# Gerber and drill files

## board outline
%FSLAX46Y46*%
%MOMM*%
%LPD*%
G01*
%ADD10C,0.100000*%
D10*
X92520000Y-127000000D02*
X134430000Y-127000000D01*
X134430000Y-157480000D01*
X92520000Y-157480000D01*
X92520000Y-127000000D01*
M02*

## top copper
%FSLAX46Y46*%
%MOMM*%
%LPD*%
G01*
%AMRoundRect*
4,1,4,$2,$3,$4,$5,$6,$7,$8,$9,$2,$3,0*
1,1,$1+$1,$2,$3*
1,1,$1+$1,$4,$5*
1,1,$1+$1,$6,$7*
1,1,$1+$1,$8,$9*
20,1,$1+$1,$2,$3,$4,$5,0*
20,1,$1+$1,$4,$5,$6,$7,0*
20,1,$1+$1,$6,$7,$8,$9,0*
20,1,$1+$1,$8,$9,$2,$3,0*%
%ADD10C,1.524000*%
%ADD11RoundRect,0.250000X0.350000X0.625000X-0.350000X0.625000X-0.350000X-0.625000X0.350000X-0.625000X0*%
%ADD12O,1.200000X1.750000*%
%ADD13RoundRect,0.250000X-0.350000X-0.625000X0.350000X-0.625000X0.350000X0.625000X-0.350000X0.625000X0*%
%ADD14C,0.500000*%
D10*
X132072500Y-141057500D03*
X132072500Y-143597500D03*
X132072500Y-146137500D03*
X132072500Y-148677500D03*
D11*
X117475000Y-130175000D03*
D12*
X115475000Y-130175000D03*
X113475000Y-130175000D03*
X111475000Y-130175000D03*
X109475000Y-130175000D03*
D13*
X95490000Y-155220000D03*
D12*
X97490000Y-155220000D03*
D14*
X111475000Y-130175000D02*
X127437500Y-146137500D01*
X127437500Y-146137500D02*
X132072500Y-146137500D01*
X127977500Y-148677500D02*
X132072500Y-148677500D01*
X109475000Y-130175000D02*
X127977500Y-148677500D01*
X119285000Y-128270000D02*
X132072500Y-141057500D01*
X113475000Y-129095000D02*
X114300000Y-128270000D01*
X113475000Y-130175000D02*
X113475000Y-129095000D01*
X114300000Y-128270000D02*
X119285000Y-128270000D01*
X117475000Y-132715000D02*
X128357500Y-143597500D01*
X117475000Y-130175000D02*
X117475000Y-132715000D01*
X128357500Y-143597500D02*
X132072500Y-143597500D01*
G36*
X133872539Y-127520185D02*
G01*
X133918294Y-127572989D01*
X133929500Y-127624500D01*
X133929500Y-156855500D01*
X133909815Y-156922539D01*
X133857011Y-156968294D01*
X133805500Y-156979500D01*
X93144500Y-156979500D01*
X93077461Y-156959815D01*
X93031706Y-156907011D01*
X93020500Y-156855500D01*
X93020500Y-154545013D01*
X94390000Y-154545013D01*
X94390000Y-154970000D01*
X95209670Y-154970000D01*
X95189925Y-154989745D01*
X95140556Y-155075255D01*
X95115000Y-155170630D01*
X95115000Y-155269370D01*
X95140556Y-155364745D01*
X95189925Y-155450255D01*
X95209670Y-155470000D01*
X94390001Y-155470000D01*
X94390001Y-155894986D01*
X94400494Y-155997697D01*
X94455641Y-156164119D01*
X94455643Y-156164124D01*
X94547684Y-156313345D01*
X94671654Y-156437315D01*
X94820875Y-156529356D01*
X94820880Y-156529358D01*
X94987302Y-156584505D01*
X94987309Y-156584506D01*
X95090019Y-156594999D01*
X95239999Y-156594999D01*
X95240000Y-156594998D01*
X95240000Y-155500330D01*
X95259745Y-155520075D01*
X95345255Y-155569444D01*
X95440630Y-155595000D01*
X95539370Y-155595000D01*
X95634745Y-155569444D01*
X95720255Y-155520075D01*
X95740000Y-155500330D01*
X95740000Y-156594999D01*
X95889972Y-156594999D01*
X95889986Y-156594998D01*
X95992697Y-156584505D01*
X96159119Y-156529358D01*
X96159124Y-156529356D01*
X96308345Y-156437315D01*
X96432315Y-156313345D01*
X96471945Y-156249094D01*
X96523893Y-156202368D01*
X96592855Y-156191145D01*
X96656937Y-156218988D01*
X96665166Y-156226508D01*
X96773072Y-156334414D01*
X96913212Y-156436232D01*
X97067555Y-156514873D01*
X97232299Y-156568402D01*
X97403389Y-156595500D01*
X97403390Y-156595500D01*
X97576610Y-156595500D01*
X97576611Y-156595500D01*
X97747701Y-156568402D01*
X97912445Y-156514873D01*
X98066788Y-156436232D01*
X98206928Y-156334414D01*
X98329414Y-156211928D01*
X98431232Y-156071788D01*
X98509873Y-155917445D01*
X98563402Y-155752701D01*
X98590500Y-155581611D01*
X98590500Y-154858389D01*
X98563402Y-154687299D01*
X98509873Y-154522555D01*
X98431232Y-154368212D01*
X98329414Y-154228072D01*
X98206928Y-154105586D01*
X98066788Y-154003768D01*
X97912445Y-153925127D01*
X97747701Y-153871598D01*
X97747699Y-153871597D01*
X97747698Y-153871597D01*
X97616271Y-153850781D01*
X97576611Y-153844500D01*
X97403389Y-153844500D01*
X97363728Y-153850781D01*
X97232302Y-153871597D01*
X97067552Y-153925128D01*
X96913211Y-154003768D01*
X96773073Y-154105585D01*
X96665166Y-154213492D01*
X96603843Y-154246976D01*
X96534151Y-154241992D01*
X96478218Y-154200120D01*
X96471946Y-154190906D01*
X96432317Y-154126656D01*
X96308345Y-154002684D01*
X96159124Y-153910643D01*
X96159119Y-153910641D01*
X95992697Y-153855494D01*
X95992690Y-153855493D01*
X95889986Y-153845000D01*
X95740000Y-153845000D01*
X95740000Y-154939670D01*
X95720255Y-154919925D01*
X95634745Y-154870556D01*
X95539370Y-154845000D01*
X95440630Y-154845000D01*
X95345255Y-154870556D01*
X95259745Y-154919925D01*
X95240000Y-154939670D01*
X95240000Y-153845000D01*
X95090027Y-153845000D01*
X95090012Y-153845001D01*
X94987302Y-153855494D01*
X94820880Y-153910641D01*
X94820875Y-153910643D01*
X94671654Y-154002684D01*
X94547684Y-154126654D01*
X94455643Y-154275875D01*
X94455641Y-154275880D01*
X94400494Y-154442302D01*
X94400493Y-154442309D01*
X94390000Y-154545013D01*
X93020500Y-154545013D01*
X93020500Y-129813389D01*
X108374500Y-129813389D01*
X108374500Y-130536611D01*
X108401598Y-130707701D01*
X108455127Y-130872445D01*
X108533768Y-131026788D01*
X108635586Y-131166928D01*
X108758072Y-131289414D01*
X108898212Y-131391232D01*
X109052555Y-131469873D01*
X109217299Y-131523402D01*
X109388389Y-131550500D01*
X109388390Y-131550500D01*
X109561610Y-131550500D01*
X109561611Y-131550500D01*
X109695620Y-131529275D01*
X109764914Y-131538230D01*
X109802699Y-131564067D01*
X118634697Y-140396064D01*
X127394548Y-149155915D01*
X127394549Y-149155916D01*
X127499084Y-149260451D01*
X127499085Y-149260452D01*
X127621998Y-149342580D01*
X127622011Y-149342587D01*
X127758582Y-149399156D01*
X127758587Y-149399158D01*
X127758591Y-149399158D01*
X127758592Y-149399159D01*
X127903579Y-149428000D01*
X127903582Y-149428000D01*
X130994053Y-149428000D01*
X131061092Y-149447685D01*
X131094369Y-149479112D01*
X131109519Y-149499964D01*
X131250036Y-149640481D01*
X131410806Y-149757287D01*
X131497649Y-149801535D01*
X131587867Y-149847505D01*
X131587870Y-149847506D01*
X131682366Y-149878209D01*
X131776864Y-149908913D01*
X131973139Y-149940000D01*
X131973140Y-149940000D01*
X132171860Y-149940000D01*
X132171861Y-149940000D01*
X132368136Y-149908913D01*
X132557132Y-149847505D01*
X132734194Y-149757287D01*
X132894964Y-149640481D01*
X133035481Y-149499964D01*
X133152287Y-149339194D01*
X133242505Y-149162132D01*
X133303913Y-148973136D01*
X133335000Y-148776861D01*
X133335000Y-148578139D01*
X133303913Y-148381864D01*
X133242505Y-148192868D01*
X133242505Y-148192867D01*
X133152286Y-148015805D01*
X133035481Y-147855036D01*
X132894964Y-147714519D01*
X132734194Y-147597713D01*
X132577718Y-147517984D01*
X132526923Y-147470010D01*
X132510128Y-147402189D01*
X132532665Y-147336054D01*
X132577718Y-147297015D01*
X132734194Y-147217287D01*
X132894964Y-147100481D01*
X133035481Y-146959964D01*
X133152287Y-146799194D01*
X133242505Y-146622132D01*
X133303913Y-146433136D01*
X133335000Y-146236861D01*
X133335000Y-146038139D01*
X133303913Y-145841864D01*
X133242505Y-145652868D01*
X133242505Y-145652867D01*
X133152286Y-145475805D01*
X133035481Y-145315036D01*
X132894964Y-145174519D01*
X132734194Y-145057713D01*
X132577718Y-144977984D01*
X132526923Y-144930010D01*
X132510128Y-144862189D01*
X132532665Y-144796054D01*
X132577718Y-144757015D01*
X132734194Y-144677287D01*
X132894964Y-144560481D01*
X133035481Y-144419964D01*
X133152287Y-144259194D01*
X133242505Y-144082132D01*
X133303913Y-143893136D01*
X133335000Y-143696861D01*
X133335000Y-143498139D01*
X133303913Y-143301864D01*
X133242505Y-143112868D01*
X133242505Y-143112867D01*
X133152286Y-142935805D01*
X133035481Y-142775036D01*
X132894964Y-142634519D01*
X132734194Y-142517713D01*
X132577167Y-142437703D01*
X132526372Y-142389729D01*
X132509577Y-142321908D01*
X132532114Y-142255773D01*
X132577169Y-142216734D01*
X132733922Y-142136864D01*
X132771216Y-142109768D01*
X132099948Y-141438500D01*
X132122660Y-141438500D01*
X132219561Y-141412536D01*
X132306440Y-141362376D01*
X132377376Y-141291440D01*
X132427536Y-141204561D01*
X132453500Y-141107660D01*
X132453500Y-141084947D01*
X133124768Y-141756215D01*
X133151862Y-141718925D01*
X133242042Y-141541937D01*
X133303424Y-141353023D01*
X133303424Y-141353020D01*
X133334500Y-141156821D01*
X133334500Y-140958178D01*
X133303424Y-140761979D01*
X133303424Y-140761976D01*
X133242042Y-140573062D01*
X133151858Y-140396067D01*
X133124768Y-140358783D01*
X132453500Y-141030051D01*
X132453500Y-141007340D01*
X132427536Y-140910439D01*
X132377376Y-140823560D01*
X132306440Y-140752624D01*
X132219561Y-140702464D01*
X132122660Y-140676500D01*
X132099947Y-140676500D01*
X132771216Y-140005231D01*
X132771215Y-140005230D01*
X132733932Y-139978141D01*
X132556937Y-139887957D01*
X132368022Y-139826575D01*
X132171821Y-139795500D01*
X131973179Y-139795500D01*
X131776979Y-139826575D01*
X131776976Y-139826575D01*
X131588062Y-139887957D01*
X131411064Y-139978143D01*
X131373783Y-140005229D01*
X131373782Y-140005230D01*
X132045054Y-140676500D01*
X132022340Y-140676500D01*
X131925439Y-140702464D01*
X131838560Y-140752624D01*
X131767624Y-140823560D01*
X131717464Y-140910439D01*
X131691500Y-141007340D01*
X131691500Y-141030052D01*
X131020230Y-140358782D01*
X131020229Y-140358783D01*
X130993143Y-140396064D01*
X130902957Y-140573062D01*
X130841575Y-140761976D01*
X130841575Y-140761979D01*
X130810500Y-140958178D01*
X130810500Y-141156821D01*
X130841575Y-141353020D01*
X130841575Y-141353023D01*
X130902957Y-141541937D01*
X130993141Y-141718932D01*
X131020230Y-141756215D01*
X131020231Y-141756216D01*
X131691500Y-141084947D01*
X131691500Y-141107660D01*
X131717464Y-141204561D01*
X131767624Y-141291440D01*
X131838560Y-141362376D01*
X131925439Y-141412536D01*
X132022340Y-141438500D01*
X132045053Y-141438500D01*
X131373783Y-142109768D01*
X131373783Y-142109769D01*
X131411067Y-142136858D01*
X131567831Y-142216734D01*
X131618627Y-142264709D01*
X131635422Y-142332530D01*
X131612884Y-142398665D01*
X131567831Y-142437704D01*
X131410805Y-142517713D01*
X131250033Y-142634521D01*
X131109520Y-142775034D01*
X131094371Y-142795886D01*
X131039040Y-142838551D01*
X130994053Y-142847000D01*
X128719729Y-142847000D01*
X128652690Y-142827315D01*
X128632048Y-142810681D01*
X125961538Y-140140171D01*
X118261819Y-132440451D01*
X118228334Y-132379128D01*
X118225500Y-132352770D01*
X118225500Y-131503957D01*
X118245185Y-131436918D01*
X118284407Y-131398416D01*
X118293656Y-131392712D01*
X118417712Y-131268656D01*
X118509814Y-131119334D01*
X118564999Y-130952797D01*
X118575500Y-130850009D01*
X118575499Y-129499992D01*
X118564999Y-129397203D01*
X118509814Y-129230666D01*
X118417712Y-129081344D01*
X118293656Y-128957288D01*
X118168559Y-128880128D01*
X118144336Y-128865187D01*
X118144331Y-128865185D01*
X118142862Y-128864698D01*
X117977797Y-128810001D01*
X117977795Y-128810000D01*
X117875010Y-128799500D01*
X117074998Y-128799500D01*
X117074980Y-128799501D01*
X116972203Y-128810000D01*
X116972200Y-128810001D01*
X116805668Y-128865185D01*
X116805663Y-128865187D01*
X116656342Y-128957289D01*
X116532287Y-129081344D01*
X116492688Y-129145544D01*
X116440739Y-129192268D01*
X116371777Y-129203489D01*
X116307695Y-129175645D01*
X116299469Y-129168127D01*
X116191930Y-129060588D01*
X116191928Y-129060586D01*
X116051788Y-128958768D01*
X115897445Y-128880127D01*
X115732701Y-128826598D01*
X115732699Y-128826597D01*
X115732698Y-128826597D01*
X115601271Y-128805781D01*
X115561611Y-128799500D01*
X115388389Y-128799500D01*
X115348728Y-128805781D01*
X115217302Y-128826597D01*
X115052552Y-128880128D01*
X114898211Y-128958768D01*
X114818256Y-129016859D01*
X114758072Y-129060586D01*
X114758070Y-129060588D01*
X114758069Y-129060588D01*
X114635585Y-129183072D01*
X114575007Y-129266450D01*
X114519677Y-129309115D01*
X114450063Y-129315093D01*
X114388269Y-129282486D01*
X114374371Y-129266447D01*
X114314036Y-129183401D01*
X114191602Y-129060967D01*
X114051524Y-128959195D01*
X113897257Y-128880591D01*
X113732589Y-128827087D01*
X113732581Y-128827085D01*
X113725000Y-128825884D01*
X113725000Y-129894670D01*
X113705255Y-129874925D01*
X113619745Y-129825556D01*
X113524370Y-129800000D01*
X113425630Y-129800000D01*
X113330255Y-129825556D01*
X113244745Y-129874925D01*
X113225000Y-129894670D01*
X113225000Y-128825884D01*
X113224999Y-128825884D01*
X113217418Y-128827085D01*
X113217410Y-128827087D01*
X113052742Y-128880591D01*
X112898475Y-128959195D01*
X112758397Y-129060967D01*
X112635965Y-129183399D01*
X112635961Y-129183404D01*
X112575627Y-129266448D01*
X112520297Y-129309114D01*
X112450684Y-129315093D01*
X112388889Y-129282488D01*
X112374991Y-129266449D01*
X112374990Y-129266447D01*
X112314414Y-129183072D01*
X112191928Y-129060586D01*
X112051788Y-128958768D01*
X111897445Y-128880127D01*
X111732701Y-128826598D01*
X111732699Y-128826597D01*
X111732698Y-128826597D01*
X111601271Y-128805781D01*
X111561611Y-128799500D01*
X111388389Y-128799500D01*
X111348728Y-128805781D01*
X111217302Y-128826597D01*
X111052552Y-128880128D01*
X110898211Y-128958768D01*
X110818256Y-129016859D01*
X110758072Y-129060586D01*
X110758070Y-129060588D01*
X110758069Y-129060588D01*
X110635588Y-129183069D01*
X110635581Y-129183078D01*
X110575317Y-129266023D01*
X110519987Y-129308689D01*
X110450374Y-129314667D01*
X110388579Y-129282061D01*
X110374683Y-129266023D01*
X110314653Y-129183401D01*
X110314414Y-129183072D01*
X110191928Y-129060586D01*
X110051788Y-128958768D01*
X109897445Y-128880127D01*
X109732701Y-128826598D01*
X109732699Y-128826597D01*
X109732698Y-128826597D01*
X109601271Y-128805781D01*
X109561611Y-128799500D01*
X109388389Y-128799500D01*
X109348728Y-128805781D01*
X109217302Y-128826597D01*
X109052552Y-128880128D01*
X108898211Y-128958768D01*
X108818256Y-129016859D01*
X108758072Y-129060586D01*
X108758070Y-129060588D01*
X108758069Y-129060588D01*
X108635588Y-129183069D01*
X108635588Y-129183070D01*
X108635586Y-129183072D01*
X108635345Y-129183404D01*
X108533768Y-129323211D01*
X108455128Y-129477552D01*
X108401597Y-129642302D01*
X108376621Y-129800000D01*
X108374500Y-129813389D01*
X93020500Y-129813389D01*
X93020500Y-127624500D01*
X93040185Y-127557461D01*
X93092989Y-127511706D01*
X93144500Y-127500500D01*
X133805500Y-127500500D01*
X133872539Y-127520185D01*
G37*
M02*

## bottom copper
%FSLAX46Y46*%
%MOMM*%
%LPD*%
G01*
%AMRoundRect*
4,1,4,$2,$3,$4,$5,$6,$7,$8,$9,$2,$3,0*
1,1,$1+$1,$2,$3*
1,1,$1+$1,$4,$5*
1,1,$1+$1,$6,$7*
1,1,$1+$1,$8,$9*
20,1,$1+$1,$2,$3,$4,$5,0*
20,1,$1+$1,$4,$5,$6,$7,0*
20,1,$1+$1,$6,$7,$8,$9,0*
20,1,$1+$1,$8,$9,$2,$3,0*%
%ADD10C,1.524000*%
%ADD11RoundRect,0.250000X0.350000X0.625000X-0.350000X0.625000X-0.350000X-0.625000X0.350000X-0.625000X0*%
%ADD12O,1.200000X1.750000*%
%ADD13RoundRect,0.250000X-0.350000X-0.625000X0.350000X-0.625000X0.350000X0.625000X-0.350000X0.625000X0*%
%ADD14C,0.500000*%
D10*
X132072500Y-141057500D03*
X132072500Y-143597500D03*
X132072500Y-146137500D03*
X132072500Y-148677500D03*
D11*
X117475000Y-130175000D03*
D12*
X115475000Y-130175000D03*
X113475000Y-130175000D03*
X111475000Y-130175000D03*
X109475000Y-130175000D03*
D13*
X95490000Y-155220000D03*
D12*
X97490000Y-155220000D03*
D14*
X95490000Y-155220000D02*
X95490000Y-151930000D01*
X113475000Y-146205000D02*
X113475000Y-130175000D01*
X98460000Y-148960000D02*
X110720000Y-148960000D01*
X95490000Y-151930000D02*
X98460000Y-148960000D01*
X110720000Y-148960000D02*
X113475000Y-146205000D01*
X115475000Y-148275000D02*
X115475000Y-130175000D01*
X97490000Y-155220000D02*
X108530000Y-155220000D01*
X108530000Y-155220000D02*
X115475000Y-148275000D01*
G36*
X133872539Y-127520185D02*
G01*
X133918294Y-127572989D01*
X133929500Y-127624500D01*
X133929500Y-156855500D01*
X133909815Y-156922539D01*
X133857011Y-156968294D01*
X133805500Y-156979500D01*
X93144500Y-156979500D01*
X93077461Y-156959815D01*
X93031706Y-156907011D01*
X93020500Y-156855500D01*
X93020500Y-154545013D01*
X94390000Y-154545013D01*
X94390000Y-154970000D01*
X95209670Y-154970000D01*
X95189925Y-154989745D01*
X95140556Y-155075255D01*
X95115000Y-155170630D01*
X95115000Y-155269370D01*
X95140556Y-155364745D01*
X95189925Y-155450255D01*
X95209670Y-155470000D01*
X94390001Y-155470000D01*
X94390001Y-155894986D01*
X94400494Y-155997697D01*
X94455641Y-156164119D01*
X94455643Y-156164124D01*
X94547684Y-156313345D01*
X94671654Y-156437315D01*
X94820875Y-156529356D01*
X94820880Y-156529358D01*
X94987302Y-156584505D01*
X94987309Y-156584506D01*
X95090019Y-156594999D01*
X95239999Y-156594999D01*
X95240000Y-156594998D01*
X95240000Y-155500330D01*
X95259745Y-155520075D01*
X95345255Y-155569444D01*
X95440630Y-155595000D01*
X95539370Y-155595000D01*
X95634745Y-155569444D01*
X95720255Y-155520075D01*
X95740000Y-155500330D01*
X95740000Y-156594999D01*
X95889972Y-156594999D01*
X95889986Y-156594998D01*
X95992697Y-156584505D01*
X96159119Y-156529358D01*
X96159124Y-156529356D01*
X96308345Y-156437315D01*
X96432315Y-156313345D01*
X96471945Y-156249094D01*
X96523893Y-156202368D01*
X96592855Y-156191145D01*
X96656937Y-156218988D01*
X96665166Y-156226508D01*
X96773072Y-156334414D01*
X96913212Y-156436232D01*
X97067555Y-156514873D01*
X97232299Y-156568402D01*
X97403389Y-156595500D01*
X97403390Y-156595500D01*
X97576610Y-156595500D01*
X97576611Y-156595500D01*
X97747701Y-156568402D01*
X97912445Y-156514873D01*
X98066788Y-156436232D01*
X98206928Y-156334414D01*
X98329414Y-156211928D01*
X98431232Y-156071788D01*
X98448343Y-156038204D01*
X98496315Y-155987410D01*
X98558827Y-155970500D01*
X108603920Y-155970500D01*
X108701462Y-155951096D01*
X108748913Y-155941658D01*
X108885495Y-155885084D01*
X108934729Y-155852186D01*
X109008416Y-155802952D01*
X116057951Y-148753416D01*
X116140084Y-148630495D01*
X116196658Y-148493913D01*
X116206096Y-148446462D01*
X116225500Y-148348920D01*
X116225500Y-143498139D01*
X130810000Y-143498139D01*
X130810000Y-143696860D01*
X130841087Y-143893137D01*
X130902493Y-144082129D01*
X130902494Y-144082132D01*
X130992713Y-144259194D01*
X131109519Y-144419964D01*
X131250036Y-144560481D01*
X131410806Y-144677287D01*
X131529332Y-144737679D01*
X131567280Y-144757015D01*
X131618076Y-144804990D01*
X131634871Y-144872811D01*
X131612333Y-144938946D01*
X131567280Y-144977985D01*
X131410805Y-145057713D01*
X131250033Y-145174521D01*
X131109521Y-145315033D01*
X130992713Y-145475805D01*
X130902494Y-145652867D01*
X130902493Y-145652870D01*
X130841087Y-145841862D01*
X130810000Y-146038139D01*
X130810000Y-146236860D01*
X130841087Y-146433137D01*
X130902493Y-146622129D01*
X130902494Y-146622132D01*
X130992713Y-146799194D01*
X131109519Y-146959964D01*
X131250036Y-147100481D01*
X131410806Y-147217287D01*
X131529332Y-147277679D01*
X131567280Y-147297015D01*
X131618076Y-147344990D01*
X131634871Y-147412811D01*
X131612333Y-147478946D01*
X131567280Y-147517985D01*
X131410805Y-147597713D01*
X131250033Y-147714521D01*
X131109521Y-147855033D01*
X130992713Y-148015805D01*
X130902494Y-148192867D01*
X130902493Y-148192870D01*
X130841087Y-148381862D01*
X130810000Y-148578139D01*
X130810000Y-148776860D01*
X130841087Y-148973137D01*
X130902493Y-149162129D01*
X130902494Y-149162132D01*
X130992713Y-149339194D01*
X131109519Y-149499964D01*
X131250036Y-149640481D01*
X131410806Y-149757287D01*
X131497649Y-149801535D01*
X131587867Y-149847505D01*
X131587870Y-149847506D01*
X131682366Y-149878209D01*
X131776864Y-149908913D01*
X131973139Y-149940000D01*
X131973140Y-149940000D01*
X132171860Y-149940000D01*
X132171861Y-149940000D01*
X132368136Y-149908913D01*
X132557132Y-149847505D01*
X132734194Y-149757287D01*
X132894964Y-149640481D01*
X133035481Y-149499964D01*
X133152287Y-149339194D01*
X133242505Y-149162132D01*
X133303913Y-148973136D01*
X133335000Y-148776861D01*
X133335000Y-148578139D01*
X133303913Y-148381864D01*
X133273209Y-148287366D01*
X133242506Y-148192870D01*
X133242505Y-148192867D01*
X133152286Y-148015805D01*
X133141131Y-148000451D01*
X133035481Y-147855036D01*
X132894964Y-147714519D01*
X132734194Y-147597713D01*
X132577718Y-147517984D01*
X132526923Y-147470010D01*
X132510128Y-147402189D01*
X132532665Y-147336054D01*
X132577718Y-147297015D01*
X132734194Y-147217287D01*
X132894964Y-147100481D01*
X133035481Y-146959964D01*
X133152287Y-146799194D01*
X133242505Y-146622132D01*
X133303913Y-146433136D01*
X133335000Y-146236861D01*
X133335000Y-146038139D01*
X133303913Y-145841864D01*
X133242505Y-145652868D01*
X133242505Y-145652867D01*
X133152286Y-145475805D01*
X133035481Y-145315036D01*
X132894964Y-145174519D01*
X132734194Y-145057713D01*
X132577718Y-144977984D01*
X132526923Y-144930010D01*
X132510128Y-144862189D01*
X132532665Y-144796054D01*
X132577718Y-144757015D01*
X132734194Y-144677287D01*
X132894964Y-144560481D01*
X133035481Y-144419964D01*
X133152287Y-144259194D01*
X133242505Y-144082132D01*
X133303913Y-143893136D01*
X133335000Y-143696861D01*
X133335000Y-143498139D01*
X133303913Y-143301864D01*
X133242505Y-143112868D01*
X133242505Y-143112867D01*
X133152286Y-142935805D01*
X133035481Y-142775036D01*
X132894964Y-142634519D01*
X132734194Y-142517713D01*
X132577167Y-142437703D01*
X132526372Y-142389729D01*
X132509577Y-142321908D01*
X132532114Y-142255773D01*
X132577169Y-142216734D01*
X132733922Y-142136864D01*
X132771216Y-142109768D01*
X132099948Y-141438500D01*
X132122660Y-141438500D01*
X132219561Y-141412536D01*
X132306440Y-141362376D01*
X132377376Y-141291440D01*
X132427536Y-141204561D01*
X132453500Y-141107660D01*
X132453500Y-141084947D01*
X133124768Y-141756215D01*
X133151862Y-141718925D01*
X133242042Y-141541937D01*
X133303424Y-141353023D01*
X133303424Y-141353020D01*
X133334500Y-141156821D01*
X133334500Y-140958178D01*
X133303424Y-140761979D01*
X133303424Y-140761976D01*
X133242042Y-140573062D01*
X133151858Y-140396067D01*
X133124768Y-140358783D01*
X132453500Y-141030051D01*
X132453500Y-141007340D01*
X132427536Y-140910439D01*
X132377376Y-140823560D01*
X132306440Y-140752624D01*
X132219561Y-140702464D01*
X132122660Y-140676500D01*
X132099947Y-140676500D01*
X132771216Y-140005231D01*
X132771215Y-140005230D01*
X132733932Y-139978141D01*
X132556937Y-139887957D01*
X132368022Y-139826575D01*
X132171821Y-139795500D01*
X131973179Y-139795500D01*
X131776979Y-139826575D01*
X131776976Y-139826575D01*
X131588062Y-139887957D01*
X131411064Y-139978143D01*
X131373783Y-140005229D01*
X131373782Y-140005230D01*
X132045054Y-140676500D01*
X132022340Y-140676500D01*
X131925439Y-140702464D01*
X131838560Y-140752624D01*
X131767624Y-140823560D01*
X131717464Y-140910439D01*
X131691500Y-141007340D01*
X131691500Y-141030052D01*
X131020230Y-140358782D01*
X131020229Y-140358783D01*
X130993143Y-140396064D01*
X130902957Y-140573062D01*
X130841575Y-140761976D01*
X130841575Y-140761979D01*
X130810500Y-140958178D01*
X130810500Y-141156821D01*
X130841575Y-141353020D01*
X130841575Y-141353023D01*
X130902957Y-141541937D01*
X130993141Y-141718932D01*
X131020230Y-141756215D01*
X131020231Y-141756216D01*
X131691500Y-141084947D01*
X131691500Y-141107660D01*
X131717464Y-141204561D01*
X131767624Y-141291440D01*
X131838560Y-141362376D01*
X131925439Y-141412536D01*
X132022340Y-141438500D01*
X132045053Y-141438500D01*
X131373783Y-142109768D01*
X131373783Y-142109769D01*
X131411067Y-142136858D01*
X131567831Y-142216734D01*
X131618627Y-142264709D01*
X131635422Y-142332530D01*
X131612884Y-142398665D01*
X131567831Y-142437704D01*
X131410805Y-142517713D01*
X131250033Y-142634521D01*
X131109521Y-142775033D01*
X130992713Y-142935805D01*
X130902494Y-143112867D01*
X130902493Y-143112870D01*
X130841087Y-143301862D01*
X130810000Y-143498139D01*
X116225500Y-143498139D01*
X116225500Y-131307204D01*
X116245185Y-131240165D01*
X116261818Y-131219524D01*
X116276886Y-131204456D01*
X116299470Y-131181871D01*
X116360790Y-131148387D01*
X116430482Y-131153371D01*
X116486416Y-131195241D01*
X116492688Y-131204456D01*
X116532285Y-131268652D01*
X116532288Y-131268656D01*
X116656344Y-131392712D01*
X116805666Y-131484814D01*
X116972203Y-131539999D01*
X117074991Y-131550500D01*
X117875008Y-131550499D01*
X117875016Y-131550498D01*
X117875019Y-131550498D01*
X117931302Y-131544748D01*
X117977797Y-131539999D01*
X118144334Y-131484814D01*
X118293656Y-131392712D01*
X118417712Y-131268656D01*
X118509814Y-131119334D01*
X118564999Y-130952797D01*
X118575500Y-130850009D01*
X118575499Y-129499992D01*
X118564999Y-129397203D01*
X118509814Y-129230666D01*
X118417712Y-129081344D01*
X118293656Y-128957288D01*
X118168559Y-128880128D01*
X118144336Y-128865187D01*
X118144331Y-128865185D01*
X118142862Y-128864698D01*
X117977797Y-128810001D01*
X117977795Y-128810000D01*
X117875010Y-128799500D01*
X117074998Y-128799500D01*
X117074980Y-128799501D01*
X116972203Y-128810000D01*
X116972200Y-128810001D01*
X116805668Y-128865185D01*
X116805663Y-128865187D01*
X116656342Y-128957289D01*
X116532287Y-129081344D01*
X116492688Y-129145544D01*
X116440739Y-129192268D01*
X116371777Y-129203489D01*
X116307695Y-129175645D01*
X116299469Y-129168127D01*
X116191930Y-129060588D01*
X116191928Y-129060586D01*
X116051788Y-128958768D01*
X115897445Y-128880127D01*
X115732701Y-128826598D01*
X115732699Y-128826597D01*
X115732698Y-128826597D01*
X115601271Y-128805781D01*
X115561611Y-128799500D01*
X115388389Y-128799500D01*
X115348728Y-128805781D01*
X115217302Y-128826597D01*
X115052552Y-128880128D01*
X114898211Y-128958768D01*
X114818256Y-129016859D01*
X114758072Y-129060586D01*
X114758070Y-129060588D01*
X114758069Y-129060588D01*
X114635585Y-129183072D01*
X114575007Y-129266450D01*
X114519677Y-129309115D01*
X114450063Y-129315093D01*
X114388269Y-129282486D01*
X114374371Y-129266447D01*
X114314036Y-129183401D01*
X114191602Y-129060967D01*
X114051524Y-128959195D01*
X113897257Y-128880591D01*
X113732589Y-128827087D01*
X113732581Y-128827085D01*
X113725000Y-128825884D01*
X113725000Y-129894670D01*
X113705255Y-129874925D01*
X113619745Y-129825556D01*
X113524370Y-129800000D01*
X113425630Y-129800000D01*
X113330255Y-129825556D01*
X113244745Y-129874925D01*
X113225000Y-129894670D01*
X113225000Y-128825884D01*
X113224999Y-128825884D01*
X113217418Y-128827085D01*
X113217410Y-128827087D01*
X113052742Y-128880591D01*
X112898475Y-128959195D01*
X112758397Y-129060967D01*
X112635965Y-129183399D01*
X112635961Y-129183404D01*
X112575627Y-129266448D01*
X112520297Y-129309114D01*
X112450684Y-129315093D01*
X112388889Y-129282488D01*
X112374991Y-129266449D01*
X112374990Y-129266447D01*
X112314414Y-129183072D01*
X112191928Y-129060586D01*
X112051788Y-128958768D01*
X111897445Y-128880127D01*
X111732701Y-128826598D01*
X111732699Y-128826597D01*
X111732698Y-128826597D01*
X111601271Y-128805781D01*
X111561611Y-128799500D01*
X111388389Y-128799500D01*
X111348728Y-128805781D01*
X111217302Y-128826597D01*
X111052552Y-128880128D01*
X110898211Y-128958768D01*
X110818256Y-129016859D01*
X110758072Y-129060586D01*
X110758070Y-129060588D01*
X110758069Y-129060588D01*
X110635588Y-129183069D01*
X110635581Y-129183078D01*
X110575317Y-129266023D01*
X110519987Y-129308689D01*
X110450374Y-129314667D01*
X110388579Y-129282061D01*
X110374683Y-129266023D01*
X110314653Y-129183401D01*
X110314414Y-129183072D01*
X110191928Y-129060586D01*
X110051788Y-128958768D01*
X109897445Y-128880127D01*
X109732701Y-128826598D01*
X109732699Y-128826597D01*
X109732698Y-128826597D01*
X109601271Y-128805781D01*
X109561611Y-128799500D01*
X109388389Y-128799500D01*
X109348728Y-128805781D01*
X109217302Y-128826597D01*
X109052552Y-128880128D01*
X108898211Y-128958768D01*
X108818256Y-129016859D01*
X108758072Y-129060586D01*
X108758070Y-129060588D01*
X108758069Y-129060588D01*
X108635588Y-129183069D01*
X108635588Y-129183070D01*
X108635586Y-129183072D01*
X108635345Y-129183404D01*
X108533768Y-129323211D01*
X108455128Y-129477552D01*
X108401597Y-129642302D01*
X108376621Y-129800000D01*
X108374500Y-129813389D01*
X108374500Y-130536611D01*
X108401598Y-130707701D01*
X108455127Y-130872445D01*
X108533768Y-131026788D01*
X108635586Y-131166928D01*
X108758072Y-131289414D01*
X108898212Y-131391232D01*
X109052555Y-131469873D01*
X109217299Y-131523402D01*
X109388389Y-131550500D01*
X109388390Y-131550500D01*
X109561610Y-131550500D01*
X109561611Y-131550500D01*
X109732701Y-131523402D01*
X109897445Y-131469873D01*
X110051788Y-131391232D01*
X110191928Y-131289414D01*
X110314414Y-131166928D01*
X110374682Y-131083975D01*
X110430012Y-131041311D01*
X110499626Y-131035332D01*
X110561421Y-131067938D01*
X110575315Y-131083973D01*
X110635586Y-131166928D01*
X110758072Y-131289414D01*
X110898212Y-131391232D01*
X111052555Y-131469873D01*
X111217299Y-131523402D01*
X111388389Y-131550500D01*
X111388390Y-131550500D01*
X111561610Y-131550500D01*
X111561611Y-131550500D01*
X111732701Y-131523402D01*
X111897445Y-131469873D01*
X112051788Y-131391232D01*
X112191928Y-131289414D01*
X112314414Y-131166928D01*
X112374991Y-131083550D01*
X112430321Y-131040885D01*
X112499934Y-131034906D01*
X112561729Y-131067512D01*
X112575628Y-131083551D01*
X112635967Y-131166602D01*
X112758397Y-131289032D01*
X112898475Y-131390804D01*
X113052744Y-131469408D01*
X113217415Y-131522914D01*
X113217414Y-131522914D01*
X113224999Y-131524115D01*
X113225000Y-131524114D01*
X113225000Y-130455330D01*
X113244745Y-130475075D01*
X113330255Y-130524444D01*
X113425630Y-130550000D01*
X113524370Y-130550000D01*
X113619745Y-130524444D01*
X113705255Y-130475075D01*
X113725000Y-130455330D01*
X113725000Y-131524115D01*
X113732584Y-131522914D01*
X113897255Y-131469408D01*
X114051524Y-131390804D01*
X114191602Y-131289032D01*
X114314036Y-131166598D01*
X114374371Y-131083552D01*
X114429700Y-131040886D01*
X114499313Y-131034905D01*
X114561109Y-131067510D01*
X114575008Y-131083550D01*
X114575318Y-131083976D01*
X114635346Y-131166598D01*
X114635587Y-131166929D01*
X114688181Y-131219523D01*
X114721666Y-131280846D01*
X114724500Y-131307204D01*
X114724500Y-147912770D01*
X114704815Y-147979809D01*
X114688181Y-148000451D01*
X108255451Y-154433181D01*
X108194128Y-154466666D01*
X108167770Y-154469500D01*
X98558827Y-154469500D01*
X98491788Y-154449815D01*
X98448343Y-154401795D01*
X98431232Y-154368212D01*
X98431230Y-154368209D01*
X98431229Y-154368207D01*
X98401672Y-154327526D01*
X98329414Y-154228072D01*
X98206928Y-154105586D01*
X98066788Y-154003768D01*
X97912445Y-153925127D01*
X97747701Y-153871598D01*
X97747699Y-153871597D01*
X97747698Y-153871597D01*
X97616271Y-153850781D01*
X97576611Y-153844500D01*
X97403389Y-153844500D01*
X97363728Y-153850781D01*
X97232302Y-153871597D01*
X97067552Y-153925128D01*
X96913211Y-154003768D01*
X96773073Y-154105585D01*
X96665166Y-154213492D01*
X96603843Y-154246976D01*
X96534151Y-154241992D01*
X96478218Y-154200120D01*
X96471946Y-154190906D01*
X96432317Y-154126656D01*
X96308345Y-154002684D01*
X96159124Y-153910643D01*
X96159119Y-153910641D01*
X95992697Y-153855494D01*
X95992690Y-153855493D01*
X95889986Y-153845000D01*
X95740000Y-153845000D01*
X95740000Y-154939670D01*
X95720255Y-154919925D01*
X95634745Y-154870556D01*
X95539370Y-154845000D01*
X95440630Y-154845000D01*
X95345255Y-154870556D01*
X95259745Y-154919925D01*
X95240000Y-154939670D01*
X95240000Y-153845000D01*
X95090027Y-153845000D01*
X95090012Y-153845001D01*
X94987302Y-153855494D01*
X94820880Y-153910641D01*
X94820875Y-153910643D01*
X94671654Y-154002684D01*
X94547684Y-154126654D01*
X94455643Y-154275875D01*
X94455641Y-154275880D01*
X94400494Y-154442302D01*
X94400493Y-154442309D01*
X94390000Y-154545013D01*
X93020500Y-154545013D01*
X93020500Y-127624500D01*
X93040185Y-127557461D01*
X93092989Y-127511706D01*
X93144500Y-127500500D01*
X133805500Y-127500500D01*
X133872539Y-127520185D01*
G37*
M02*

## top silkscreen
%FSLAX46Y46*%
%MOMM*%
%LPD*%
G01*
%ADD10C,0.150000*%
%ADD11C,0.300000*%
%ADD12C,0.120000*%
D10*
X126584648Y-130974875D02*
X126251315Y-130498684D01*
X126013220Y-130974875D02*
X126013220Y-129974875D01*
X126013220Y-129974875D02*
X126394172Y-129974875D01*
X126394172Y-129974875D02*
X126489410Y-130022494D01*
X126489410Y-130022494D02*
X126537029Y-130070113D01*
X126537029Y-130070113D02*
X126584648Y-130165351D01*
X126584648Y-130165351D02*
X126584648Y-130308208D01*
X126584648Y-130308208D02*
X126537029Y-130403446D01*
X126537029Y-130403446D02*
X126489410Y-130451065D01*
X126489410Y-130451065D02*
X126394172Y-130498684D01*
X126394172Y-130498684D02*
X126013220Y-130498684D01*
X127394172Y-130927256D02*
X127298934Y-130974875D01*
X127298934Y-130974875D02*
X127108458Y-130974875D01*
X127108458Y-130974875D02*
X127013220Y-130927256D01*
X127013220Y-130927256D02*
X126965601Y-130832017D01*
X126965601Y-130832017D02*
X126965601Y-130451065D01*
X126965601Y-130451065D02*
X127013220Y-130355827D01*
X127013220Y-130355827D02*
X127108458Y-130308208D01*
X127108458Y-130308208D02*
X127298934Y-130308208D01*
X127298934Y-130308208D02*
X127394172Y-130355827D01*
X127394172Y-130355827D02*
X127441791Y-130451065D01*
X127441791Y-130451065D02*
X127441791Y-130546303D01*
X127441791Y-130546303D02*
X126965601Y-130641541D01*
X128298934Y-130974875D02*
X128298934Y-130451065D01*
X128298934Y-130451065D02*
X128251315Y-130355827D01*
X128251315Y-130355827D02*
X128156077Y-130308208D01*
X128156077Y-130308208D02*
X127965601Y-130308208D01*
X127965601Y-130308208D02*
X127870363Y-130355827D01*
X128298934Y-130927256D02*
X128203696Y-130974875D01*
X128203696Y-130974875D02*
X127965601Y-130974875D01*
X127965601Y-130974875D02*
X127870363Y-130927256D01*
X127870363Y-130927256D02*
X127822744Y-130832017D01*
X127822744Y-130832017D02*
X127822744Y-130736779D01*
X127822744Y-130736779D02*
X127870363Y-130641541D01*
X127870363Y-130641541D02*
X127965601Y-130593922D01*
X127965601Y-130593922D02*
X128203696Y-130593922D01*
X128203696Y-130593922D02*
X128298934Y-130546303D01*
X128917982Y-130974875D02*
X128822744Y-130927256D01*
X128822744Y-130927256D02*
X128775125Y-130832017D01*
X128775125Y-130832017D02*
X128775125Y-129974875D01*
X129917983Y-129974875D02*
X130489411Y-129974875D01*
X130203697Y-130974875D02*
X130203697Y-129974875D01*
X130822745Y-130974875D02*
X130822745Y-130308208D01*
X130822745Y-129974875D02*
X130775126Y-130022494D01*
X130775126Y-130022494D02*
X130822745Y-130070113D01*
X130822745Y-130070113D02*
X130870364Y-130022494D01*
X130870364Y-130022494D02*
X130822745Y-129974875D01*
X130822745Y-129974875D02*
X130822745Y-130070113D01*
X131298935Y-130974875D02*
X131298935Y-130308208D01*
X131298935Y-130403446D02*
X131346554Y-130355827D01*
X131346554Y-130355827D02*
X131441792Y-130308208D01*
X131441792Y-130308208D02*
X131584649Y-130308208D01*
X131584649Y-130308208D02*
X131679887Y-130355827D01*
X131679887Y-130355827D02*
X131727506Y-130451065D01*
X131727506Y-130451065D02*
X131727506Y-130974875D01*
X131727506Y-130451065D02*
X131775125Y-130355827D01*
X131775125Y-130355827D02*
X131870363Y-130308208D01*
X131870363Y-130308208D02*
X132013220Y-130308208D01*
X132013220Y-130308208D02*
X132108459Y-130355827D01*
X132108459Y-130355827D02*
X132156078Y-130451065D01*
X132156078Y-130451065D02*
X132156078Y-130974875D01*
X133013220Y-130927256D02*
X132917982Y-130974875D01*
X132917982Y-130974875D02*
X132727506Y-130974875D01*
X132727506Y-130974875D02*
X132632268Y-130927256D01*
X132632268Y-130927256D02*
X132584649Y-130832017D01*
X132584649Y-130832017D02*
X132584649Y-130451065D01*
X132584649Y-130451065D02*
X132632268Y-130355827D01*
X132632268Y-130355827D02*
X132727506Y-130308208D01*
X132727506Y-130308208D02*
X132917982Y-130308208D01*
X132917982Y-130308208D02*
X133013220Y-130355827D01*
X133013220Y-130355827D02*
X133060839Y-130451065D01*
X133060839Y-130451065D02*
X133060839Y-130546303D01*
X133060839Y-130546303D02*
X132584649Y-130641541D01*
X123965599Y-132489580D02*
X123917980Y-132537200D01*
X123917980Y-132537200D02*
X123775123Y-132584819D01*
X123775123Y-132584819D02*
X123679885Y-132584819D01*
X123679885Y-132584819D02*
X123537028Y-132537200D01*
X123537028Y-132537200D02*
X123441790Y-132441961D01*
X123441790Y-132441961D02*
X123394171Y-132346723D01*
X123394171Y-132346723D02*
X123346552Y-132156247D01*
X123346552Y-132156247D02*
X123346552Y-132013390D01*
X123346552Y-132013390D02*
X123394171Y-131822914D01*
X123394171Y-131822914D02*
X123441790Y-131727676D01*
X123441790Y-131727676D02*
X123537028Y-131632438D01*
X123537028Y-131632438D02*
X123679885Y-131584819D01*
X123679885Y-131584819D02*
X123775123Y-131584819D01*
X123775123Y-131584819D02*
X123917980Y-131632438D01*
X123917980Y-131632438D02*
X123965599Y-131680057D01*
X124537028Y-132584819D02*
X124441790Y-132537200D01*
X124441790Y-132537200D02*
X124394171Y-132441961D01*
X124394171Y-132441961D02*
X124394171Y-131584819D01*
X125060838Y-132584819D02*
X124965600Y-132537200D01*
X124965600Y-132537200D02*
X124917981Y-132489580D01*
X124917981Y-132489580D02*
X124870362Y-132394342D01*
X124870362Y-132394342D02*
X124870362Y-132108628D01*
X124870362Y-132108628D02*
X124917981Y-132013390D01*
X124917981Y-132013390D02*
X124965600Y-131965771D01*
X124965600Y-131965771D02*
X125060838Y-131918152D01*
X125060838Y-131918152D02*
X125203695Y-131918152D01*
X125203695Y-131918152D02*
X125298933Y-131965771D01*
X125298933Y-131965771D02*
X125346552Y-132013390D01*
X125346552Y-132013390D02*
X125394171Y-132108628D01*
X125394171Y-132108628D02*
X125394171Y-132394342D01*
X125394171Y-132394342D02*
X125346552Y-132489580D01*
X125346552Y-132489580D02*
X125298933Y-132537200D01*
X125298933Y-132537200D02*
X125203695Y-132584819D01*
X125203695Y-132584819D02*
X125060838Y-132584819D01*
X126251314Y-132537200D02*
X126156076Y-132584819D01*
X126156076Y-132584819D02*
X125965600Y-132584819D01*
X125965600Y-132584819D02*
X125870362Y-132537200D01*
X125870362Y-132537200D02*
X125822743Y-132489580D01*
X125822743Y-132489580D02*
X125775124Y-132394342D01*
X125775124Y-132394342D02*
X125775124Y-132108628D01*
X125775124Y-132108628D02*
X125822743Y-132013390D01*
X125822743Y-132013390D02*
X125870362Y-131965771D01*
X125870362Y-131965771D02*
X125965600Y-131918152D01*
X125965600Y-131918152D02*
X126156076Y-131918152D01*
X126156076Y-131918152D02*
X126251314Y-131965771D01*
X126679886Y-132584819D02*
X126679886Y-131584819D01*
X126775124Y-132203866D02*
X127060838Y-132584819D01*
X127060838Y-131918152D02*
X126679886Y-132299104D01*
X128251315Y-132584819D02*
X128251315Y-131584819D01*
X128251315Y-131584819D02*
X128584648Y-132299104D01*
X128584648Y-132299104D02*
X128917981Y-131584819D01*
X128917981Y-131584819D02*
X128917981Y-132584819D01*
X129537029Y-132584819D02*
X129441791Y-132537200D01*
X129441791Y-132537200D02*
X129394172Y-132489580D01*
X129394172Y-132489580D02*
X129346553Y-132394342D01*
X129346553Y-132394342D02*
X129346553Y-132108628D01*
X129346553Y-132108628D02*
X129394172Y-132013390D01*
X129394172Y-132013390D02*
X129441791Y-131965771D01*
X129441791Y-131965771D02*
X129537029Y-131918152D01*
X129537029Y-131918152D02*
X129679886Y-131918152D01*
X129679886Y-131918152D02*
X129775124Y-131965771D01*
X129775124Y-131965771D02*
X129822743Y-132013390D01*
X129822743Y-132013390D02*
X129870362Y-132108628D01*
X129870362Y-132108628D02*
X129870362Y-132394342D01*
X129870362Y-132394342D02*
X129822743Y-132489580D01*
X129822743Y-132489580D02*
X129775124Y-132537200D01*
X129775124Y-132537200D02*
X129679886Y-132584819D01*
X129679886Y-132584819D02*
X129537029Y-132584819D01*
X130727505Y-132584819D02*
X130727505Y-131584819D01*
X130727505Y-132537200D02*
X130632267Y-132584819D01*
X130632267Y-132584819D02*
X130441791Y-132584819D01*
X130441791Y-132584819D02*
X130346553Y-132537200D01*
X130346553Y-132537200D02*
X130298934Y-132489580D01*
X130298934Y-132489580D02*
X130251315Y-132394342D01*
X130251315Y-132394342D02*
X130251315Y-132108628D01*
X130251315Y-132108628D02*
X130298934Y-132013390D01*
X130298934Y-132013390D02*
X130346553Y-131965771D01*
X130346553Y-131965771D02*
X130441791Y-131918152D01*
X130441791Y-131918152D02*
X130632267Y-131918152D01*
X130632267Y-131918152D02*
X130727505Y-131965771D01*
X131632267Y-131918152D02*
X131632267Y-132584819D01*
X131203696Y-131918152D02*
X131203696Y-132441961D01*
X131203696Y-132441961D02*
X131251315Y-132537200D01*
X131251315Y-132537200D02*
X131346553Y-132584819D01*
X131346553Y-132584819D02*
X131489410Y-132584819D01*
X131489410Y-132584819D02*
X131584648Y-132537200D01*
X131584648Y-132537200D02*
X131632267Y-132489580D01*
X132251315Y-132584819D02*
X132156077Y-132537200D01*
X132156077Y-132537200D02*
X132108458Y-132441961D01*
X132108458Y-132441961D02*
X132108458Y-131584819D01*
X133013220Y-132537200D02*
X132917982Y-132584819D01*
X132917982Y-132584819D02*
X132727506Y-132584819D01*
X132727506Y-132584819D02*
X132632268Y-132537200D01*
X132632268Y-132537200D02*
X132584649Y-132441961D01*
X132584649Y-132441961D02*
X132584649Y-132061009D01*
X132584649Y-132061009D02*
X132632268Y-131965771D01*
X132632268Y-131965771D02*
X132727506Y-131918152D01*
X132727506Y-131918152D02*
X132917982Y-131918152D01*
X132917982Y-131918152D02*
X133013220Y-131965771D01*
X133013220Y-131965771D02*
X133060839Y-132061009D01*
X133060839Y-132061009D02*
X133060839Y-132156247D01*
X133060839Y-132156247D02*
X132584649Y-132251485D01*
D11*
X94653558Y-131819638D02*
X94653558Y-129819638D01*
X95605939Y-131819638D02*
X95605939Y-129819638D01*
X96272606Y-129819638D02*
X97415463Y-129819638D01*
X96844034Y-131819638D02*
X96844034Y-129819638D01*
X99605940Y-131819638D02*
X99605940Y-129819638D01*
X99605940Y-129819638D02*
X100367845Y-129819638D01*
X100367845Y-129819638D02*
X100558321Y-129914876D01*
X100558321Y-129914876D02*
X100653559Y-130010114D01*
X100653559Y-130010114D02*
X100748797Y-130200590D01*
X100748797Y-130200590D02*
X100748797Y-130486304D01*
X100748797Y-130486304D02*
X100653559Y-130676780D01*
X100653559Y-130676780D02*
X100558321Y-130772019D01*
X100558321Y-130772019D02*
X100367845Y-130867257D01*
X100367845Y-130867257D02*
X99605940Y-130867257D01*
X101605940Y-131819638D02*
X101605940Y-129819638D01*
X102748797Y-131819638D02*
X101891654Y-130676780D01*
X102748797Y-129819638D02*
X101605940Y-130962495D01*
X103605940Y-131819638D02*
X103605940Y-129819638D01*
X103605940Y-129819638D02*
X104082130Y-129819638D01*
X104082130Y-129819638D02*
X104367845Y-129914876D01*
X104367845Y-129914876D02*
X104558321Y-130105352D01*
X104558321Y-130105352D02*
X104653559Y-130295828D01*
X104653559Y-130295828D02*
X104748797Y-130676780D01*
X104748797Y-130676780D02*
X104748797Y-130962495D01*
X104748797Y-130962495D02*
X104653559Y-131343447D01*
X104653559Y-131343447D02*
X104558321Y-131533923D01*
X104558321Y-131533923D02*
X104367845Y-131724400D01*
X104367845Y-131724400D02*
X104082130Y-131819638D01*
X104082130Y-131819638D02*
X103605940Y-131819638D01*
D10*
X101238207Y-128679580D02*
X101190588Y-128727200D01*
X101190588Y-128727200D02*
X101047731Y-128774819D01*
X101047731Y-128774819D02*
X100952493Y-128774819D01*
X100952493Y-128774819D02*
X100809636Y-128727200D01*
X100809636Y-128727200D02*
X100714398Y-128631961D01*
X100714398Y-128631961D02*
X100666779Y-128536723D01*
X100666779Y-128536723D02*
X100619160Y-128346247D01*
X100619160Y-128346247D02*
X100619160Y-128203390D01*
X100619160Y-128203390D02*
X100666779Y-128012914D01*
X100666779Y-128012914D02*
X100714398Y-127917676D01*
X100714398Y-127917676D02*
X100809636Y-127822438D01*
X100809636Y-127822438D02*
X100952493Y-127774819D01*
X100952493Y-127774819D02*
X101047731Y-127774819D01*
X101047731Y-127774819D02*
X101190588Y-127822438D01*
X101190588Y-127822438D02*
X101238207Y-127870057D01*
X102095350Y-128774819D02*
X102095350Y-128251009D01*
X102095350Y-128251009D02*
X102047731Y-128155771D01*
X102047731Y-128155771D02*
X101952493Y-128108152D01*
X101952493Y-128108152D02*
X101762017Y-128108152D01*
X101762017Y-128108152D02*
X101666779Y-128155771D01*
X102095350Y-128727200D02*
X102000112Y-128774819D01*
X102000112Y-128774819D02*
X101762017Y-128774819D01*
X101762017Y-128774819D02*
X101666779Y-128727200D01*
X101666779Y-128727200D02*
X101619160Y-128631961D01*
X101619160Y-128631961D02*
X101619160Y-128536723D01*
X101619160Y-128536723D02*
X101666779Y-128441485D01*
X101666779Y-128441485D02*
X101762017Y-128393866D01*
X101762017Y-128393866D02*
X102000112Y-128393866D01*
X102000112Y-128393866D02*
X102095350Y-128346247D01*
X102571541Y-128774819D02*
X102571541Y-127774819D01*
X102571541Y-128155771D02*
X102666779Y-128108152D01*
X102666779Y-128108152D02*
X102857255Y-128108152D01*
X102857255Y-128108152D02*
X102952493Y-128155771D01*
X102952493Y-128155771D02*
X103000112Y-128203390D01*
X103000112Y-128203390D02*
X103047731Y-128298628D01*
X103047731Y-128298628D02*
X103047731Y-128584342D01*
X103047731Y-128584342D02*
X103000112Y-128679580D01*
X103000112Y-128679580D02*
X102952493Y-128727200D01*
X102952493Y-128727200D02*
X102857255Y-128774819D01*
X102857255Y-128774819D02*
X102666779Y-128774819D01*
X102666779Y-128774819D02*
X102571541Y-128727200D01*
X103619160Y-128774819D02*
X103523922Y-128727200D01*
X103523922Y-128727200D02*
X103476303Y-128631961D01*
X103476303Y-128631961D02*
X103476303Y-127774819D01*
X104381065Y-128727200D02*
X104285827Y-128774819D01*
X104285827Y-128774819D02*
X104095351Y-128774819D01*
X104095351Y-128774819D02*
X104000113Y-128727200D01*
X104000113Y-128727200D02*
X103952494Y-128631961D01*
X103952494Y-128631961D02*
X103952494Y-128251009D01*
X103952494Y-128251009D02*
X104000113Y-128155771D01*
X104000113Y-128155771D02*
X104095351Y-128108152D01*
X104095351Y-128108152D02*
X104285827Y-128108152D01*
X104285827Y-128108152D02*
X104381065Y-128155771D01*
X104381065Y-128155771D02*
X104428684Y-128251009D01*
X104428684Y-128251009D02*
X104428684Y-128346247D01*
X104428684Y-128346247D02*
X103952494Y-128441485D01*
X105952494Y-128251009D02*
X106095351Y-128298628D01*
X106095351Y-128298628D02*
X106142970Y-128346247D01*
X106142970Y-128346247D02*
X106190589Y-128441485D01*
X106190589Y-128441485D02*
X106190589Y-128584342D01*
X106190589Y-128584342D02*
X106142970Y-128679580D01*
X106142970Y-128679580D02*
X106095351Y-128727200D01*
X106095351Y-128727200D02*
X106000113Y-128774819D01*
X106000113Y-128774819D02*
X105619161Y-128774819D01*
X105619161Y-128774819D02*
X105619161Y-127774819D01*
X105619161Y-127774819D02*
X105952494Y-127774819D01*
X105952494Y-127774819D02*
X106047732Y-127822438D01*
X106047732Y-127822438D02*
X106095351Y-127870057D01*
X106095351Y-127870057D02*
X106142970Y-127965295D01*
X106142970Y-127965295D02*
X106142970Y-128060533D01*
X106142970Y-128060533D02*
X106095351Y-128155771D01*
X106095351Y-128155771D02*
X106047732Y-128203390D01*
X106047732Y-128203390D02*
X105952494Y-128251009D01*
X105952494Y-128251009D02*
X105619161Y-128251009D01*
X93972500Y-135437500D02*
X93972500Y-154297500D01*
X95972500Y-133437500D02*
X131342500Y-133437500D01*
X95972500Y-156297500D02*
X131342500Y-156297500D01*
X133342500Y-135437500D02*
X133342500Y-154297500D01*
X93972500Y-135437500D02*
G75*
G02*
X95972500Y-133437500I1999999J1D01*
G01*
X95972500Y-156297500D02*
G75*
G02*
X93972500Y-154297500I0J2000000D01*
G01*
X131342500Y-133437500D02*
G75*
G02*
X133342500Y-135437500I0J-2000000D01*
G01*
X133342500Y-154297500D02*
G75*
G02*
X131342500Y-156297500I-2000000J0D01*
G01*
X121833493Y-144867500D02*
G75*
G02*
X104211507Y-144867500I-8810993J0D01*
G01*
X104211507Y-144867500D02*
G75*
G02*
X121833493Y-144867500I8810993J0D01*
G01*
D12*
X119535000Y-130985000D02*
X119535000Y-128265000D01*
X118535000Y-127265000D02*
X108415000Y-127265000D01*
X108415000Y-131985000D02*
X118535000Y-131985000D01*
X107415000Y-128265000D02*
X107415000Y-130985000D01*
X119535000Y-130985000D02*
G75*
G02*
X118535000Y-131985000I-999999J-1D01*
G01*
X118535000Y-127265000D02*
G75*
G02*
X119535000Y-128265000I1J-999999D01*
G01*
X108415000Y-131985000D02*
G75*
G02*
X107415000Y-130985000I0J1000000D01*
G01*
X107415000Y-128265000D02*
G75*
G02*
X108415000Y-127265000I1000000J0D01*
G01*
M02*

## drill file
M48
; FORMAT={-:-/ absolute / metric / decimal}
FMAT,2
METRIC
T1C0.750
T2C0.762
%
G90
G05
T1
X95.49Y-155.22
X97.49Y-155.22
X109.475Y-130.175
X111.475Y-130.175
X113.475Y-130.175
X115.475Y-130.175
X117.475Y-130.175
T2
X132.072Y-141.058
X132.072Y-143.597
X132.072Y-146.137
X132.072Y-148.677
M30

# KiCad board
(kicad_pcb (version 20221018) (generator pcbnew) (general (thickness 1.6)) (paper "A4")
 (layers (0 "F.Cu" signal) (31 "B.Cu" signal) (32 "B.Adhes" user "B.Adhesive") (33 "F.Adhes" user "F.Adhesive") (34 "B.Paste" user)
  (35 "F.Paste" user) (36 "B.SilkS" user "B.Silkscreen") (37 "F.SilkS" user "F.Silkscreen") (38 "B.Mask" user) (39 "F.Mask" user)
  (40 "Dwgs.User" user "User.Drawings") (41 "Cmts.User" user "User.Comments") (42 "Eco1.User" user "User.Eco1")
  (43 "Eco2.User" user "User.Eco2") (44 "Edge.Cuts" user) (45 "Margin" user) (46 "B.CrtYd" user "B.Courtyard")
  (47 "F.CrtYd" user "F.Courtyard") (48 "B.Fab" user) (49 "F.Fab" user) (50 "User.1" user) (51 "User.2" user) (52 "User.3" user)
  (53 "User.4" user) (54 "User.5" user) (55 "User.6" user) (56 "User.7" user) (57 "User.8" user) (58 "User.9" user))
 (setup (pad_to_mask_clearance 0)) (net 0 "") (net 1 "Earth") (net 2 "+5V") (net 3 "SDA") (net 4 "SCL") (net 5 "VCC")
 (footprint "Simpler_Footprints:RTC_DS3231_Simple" (layer "F.Cu") (at 93.9725 133.4375)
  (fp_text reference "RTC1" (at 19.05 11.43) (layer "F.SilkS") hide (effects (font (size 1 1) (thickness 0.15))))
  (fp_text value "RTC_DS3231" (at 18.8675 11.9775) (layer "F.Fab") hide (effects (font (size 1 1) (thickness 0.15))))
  (fp_line (start 0 2) (end 0 20.86) (stroke (width 0.15) (type solid)) (layer "F.SilkS"))
  (fp_line (start 2 0) (end 37.37 0) (stroke (width 0.15) (type solid)) (layer "F.SilkS"))
  (fp_line (start 2 22.86) (end 37.37 22.86) (stroke (width 0.15) (type solid)) (layer "F.SilkS"))
  (fp_line (start 39.37 2) (end 39.37 20.86) (stroke (width 0.15) (type solid)) (layer "F.SilkS"))
  (fp_arc (start 0 2) (mid 0.585786 0.585786) (end 2 0) (stroke (width 0.15) (type default)) (layer "F.SilkS"))
  (fp_arc (start 2 22.86) (mid 0.585786 22.274214) (end 0 20.86) (stroke (width 0.15) (type default)) (layer "F.SilkS"))
  (fp_arc (start 37.37 0) (mid 38.784214 0.585786) (end 39.37 2) (stroke (width 0.15) (type default)) (layer "F.SilkS"))
  (fp_arc (start 39.37 20.86) (mid 38.784214 22.274214) (end 37.37 22.86) (stroke (width 0.15) (type default)) (layer "F.SilkS"))
  (fp_circle (center 19.05 11.43) (end 27.860993 11.43) (stroke (width 0.15) (type default)) (fill none) (layer "F.SilkS"))
  (pad "1" thru_hole circle (at 38.1 7.62) (size 1.524 1.524) (drill 0.762) (layers "*.Cu" "*.Mask") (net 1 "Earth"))
  (pad "2" thru_hole circle (at 38.1 10.16) (size 1.524 1.524) (drill 0.762) (layers "*.Cu" "*.Mask") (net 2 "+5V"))
  (pad "3" thru_hole circle (at 38.1 12.7) (size 1.524 1.524) (drill 0.762) (layers "*.Cu" "*.Mask") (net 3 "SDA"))
  (pad "4" thru_hole circle (at 38.1 15.24) (size 1.524 1.524) (drill 0.762) (layers "*.Cu" "*.Mask") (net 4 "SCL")))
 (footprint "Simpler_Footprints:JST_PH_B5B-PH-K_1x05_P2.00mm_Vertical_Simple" (layer "F.Cu") (at 117.475 130.175 180)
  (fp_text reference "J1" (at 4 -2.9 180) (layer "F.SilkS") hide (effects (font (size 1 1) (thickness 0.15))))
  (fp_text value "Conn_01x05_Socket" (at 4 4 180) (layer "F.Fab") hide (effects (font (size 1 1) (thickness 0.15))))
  (fp_line (start -2.06 -0.81) (end -2.06 1.91) (stroke (width 0.12) (type solid)) (layer "F.SilkS"))
  (fp_line (start -1.06 2.91) (end 9.06 2.91) (stroke (width 0.12) (type solid)) (layer "F.SilkS"))
  (fp_line (start 9.06 -1.81) (end -1.06 -1.81) (stroke (width 0.12) (type solid)) (layer "F.SilkS"))
  (fp_line (start 10.06 1.91) (end 10.06 -0.81) (stroke (width 0.12) (type solid)) (layer "F.SilkS"))
  (fp_arc (start -2.06 -0.81) (mid -1.767107 -1.517107) (end -1.06 -1.81) (stroke (width 0.12) (type default)) (layer "F.SilkS"))
  (fp_arc (start -1.06 2.91) (mid -1.767107 2.617107) (end -2.06 1.91) (stroke (width 0.12) (type default)) (layer "F.SilkS"))
  (fp_arc (start 9.06 -1.81) (mid 9.767107 -1.517107) (end 10.06 -0.81) (stroke (width 0.12) (type default)) (layer "F.SilkS"))
  (fp_arc (start 10.06 1.91) (mid 9.767107 2.617107) (end 9.06 2.91) (stroke (width 0.12) (type default)) (layer "F.SilkS"))
  (pad "1" thru_hole roundrect (at 0 0 180) (size 1.2 1.75) (drill 0.75) (layers "*.Cu" "*.Mask") (roundrect_rratio 0.2083333333)
   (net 2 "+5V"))
  (pad "2" thru_hole oval (at 2 0 180) (size 1.2 1.75) (drill 0.75) (layers "*.Cu" "*.Mask") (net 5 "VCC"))
  (pad "3" thru_hole oval (at 4 0 180) (size 1.2 1.75) (drill 0.75) (layers "*.Cu" "*.Mask") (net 1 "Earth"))
  (pad "4" thru_hole oval (at 6 0 180) (size 1.2 1.75) (drill 0.75) (layers "*.Cu" "*.Mask") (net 3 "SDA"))
  (pad "5" thru_hole oval (at 8 0 180) (size 1.2 1.75) (drill 0.75) (layers "*.Cu" "*.Mask") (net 4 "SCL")))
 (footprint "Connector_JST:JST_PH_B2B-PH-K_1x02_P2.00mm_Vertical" (layer "F.Cu") (at 95.49 155.22)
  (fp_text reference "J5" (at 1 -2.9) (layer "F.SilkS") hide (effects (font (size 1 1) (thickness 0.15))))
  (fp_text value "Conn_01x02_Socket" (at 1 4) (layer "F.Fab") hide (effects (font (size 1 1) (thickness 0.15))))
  (pad "1" thru_hole roundrect (at 0 0) (size 1.2 1.75) (drill 0.75) (layers "*.Cu" "*.Mask") (roundrect_rratio 0.208333) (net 1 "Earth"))
  (pad "2" thru_hole oval (at 2 0) (size 1.2 1.75) (drill 0.75) (layers "*.Cu" "*.Mask") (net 5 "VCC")))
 (gr_rect (start 92.52 127) (end 134.43 157.48) (stroke (width 0.1) (type default)) (fill none) (layer "Edge.Cuts"))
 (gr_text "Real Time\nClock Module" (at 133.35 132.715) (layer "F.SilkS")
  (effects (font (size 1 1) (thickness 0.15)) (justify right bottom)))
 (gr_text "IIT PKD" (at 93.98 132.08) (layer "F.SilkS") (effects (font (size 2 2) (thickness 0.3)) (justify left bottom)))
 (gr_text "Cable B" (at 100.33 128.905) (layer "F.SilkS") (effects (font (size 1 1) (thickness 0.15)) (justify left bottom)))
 (segment (start 111.475 130.175) (end 127.4375 146.1375) (width 0.5) (layer "F.Cu") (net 3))
 (segment (start 127.4375 146.1375) (end 132.0725 146.1375) (width 0.5) (layer "F.Cu") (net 3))
 (segment (start 127.9775 148.6775) (end 132.0725 148.6775) (width 0.5) (layer "F.Cu") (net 4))
 (segment (start 109.475 130.175) (end 127.9775 148.6775) (width 0.5) (layer "F.Cu") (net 4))
 (segment (start 119.285 128.27) (end 132.0725 141.0575) (width 0.5) (layer "F.Cu") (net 1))
 (segment (start 113.475 129.095) (end 114.3 128.27) (width 0.5) (layer "F.Cu") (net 1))
 (segment (start 113.475 130.175) (end 113.475 129.095) (width 0.5) (layer "F.Cu") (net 1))
 (segment (start 114.3 128.27) (end 119.285 128.27) (width 0.5) (layer "F.Cu") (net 1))
 (segment (start 95.49 155.22) (end 95.49 151.93) (width 0.5) (layer "B.Cu") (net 1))
 (segment (start 113.475 146.205) (end 113.475 130.175) (width 0.5) (layer "B.Cu") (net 1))
 (segment (start 98.46 148.96) (end 110.72 148.96) (width 0.5) (layer "B.Cu") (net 1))
 (segment (start 95.49 151.93) (end 98.46 148.96) (width 0.5) (layer "B.Cu") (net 1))
 (segment (start 110.72 148.96) (end 113.475 146.205) (width 0.5) (layer "B.Cu") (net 1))
 (segment (start 117.475 132.715) (end 128.3575 143.5975) (width 0.5) (layer "F.Cu") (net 2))
 (segment (start 117.475 130.175) (end 117.475 132.715) (width 0.5) (layer "F.Cu") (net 2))
 (segment (start 128.3575 143.5975) (end 132.0725 143.5975) (width 0.5) (layer "F.Cu") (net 2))
 (segment (start 115.475 148.275) (end 115.475 130.175) (width 0.5) (layer "B.Cu") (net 5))
 (segment (start 97.49 155.22) (end 108.53 155.22) (width 0.5) (layer "B.Cu") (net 5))
 (segment (start 108.53 155.22) (end 115.475 148.275) (width 0.5) (layer "B.Cu") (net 5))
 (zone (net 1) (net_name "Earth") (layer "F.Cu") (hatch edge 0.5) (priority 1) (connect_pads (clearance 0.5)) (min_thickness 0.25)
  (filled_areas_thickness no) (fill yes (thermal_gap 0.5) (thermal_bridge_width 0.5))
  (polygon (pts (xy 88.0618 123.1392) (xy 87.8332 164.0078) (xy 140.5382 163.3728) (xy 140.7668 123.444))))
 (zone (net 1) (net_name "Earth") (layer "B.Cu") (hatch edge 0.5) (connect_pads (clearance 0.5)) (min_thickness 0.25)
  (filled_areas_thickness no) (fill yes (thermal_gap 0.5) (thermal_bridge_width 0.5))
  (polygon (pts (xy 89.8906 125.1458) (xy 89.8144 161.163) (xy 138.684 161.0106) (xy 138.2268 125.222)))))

